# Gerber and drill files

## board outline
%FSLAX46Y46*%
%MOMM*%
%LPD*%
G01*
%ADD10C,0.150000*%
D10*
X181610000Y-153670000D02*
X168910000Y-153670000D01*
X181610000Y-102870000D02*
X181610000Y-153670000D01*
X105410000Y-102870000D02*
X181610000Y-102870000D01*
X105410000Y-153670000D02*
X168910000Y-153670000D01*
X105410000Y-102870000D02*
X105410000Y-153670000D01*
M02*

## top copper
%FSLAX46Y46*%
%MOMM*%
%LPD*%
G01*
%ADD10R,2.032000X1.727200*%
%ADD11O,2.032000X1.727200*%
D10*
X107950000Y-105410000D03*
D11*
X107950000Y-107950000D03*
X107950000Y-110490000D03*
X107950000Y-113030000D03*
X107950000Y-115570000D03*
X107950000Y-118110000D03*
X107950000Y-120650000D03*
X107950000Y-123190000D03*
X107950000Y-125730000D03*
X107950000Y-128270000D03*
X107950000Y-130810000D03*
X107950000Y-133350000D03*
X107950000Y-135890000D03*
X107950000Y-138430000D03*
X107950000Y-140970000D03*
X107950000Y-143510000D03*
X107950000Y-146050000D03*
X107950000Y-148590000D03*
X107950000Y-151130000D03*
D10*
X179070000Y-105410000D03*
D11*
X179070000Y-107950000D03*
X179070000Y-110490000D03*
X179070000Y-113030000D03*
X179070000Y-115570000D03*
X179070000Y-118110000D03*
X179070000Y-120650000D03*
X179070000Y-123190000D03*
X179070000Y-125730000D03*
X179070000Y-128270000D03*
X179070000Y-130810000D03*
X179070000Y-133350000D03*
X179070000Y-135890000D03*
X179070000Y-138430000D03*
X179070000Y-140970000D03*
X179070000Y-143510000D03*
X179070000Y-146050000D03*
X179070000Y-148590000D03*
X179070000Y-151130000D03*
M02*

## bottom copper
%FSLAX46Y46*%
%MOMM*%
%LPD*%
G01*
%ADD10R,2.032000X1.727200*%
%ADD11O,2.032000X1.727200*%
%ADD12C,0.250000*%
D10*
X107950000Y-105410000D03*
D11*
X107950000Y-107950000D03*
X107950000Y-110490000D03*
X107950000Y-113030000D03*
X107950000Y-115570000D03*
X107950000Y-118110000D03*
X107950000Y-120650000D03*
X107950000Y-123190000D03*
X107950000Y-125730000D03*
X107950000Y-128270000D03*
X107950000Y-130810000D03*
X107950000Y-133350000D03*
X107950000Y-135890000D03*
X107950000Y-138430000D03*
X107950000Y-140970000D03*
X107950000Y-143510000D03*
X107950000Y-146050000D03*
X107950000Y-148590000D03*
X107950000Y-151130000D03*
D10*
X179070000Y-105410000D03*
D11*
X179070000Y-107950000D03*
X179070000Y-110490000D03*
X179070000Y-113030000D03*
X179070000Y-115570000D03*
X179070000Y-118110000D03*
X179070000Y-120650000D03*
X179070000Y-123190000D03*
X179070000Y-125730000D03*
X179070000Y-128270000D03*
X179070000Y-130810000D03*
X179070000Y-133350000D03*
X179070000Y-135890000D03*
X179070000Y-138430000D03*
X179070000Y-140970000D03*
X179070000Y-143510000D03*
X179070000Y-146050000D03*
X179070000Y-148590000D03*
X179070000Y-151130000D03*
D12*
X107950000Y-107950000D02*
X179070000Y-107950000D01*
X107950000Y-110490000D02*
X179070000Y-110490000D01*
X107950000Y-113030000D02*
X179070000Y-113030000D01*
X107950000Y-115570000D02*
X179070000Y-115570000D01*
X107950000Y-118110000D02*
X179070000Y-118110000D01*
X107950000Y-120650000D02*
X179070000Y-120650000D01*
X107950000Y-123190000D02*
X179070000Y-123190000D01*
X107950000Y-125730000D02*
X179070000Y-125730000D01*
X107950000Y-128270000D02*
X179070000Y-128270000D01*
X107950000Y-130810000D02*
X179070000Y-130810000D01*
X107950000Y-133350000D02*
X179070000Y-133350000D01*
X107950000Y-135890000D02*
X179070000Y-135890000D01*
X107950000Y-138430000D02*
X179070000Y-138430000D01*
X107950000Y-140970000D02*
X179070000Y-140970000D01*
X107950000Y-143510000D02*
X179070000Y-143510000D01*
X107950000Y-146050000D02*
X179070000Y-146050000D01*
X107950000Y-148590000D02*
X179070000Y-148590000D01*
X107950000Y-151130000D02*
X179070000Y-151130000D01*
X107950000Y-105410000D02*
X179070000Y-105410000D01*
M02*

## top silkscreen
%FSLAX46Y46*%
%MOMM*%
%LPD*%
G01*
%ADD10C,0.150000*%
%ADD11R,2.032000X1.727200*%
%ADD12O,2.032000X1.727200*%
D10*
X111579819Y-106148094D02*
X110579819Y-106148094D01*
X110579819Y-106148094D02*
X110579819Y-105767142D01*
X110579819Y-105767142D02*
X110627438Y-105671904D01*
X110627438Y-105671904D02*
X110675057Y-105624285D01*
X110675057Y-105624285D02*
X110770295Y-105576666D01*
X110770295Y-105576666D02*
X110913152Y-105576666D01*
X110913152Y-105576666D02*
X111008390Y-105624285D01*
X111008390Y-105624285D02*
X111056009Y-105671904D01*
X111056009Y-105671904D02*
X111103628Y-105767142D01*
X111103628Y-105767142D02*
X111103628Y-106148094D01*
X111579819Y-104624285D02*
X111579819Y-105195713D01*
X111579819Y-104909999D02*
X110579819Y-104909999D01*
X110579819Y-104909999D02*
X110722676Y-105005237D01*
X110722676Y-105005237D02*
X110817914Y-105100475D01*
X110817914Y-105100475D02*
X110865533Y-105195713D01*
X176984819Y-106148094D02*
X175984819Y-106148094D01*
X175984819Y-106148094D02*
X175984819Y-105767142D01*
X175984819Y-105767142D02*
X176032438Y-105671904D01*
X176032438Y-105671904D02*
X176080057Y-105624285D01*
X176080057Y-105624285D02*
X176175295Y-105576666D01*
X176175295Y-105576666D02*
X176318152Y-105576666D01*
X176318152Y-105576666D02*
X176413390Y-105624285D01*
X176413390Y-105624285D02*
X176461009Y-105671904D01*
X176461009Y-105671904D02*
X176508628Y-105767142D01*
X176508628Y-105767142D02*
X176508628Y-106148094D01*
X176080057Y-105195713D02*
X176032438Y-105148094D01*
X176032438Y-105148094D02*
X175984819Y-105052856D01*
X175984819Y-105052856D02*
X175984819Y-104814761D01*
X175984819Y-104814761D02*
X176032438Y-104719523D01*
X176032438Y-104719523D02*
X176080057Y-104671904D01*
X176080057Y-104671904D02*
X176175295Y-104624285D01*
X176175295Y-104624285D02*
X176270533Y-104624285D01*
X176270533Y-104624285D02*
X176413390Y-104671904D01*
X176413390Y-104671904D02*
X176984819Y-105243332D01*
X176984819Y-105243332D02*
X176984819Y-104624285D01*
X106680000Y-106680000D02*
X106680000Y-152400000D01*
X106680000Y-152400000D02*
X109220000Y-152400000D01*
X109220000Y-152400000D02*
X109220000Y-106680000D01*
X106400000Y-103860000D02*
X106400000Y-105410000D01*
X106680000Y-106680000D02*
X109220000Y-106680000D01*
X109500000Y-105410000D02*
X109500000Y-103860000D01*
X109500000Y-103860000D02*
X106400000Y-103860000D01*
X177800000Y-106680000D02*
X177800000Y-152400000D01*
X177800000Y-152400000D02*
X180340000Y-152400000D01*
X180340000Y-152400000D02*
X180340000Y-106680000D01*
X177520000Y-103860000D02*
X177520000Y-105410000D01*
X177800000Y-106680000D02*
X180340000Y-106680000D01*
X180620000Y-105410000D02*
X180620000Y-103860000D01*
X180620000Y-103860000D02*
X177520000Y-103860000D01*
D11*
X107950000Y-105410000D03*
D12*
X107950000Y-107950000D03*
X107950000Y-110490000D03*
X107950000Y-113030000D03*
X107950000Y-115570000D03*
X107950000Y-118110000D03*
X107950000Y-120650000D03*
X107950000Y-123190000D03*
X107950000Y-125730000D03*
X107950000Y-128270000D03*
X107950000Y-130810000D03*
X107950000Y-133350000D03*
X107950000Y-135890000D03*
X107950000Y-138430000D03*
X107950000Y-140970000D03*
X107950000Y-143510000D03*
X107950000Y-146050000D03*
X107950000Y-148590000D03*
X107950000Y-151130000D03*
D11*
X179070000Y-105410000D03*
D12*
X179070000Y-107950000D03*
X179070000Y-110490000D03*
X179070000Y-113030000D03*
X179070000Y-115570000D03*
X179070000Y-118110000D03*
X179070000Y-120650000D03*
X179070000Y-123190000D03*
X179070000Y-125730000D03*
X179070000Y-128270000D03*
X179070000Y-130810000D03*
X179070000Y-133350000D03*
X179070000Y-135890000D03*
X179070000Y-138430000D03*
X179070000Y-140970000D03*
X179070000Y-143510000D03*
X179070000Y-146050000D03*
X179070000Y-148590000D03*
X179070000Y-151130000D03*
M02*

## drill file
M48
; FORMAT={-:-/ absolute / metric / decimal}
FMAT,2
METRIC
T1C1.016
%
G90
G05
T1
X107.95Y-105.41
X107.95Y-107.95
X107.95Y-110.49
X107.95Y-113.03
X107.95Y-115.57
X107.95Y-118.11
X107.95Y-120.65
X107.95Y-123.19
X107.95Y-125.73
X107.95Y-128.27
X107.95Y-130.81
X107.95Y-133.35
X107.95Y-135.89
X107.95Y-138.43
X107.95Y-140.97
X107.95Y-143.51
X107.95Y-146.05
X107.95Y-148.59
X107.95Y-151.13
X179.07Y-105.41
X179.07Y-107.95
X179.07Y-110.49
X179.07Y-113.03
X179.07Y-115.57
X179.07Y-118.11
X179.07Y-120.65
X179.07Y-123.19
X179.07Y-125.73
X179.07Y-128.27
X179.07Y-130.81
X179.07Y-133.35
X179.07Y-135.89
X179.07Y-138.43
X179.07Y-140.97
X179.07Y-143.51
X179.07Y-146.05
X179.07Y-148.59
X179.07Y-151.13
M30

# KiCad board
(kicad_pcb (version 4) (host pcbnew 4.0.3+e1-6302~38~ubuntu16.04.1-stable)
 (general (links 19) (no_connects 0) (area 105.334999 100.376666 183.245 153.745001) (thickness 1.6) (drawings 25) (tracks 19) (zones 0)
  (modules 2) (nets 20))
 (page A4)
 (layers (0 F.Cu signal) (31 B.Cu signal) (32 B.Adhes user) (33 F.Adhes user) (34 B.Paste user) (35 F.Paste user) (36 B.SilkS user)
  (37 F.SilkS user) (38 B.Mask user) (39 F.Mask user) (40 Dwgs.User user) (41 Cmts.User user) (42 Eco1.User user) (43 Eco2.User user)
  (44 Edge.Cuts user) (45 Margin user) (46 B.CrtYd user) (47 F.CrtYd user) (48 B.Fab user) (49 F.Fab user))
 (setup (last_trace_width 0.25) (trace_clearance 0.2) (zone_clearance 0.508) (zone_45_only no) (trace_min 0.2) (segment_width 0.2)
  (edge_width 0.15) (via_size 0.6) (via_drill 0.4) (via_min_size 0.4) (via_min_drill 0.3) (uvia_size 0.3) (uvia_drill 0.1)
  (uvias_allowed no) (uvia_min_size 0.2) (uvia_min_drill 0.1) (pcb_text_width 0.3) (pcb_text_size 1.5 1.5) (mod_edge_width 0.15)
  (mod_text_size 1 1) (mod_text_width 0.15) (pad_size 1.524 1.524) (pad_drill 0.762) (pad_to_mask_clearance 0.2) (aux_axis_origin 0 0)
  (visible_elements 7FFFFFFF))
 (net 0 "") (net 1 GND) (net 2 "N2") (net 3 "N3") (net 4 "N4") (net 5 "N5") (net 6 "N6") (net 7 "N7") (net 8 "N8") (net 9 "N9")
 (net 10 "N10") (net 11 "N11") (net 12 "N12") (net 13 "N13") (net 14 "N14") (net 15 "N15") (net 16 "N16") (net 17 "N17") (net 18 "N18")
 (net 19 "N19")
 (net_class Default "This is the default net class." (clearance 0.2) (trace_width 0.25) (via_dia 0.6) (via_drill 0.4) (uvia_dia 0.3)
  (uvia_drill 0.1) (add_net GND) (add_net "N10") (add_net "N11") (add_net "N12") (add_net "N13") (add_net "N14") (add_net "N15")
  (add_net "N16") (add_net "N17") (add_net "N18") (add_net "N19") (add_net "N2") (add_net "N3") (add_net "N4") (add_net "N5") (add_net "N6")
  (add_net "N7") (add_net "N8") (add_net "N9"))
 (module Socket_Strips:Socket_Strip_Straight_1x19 (layer F.Cu) (at 107.95 105.41 270)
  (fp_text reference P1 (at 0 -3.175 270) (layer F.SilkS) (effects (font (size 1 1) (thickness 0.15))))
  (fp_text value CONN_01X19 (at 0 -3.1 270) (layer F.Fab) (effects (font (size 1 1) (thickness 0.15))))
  (fp_line (start 1.27 1.27) (end 46.99 1.27) (layer F.SilkS) (width 0.15))
  (fp_line (start 46.99 1.27) (end 46.99 -1.27) (layer F.SilkS) (width 0.15))
  (fp_line (start 46.99 -1.27) (end 1.27 -1.27) (layer F.SilkS) (width 0.15))
  (fp_line (start -1.55 1.55) (end 0 1.55) (layer F.SilkS) (width 0.15))
  (fp_line (start 1.27 1.27) (end 1.27 -1.27) (layer F.SilkS) (width 0.15))
  (fp_line (start 0 -1.55) (end -1.55 -1.55) (layer F.SilkS) (width 0.15))
  (fp_line (start -1.55 -1.55) (end -1.55 1.55) (layer F.SilkS) (width 0.15))
  (pad 1 thru_hole rect (at 0 0 270) (size 1.7272 2.032) (drill 1.016) (layers *.Cu *.Mask F.SilkS) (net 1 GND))
  (pad 2 thru_hole oval (at 2.54 0 270) (size 1.7272 2.032) (drill 1.016) (layers *.Cu *.Mask F.SilkS) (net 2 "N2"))
  (pad 3 thru_hole oval (at 5.08 0 270) (size 1.7272 2.032) (drill 1.016) (layers *.Cu *.Mask F.SilkS) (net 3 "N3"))
  (pad 4 thru_hole oval (at 7.62 0 270) (size 1.7272 2.032) (drill 1.016) (layers *.Cu *.Mask F.SilkS) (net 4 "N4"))
  (pad 5 thru_hole oval (at 10.16 0 270) (size 1.7272 2.032) (drill 1.016) (layers *.Cu *.Mask F.SilkS) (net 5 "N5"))
  (pad 6 thru_hole oval (at 12.7 0 270) (size 1.7272 2.032) (drill 1.016) (layers *.Cu *.Mask F.SilkS) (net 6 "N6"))
  (pad 7 thru_hole oval (at 15.24 0 270) (size 1.7272 2.032) (drill 1.016) (layers *.Cu *.Mask F.SilkS) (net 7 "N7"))
  (pad 8 thru_hole oval (at 17.78 0 270) (size 1.7272 2.032) (drill 1.016) (layers *.Cu *.Mask F.SilkS) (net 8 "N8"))
  (pad 9 thru_hole oval (at 20.32 0 270) (size 1.7272 2.032) (drill 1.016) (layers *.Cu *.Mask F.SilkS) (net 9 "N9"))
  (pad 10 thru_hole oval (at 22.86 0 270) (size 1.7272 2.032) (drill 1.016) (layers *.Cu *.Mask F.SilkS) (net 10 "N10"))
  (pad 11 thru_hole oval (at 25.4 0 270) (size 1.7272 2.032) (drill 1.016) (layers *.Cu *.Mask F.SilkS) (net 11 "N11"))
  (pad 12 thru_hole oval (at 27.94 0 270) (size 1.7272 2.032) (drill 1.016) (layers *.Cu *.Mask F.SilkS) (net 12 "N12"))
  (pad 13 thru_hole oval (at 30.48 0 270) (size 1.7272 2.032) (drill 1.016) (layers *.Cu *.Mask F.SilkS) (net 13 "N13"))
  (pad 14 thru_hole oval (at 33.02 0 270) (size 1.7272 2.032) (drill 1.016) (layers *.Cu *.Mask F.SilkS) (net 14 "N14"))
  (pad 15 thru_hole oval (at 35.56 0 270) (size 1.7272 2.032) (drill 1.016) (layers *.Cu *.Mask F.SilkS) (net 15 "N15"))
  (pad 16 thru_hole oval (at 38.1 0 270) (size 1.7272 2.032) (drill 1.016) (layers *.Cu *.Mask F.SilkS) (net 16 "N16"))
  (pad 17 thru_hole oval (at 40.64 0 270) (size 1.7272 2.032) (drill 1.016) (layers *.Cu *.Mask F.SilkS) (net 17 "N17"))
  (pad 18 thru_hole oval (at 43.18 0 270) (size 1.7272 2.032) (drill 1.016) (layers *.Cu *.Mask F.SilkS) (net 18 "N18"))
  (pad 19 thru_hole oval (at 45.72 0 270) (size 1.7272 2.032) (drill 1.016) (layers *.Cu *.Mask F.SilkS) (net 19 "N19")))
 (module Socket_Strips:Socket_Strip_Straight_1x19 (layer F.Cu) (at 179.07 105.41 270)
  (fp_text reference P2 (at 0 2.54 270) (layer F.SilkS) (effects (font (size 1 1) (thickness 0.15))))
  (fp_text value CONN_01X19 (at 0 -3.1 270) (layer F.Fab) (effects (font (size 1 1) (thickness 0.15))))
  (fp_line (start 1.27 1.27) (end 46.99 1.27) (layer F.SilkS) (width 0.15))
  (fp_line (start 46.99 1.27) (end 46.99 -1.27) (layer F.SilkS) (width 0.15))
  (fp_line (start 46.99 -1.27) (end 1.27 -1.27) (layer F.SilkS) (width 0.15))
  (fp_line (start -1.55 1.55) (end 0 1.55) (layer F.SilkS) (width 0.15))
  (fp_line (start 1.27 1.27) (end 1.27 -1.27) (layer F.SilkS) (width 0.15))
  (fp_line (start 0 -1.55) (end -1.55 -1.55) (layer F.SilkS) (width 0.15))
  (fp_line (start -1.55 -1.55) (end -1.55 1.55) (layer F.SilkS) (width 0.15))
  (pad 1 thru_hole rect (at 0 0 270) (size 1.7272 2.032) (drill 1.016) (layers *.Cu *.Mask F.SilkS) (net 1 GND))
  (pad 2 thru_hole oval (at 2.54 0 270) (size 1.7272 2.032) (drill 1.016) (layers *.Cu *.Mask F.SilkS) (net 2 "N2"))
  (pad 3 thru_hole oval (at 5.08 0 270) (size 1.7272 2.032) (drill 1.016) (layers *.Cu *.Mask F.SilkS) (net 3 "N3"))
  (pad 4 thru_hole oval (at 7.62 0 270) (size 1.7272 2.032) (drill 1.016) (layers *.Cu *.Mask F.SilkS) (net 4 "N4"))
  (pad 5 thru_hole oval (at 10.16 0 270) (size 1.7272 2.032) (drill 1.016) (layers *.Cu *.Mask F.SilkS) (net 5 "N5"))
  (pad 6 thru_hole oval (at 12.7 0 270) (size 1.7272 2.032) (drill 1.016) (layers *.Cu *.Mask F.SilkS) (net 6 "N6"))
  (pad 7 thru_hole oval (at 15.24 0 270) (size 1.7272 2.032) (drill 1.016) (layers *.Cu *.Mask F.SilkS) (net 7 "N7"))
  (pad 8 thru_hole oval (at 17.78 0 270) (size 1.7272 2.032) (drill 1.016) (layers *.Cu *.Mask F.SilkS) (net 8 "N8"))
  (pad 9 thru_hole oval (at 20.32 0 270) (size 1.7272 2.032) (drill 1.016) (layers *.Cu *.Mask F.SilkS) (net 9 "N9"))
  (pad 10 thru_hole oval (at 22.86 0 270) (size 1.7272 2.032) (drill 1.016) (layers *.Cu *.Mask F.SilkS) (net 10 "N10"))
  (pad 11 thru_hole oval (at 25.4 0 270) (size 1.7272 2.032) (drill 1.016) (layers *.Cu *.Mask F.SilkS) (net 11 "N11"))
  (pad 12 thru_hole oval (at 27.94 0 270) (size 1.7272 2.032) (drill 1.016) (layers *.Cu *.Mask F.SilkS) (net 12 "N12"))
  (pad 13 thru_hole oval (at 30.48 0 270) (size 1.7272 2.032) (drill 1.016) (layers *.Cu *.Mask F.SilkS) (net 13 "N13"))
  (pad 14 thru_hole oval (at 33.02 0 270) (size 1.7272 2.032) (drill 1.016) (layers *.Cu *.Mask F.SilkS) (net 14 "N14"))
  (pad 15 thru_hole oval (at 35.56 0 270) (size 1.7272 2.032) (drill 1.016) (layers *.Cu *.Mask F.SilkS) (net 15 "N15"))
  (pad 16 thru_hole oval (at 38.1 0 270) (size 1.7272 2.032) (drill 1.016) (layers *.Cu *.Mask F.SilkS) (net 16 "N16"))
  (pad 17 thru_hole oval (at 40.64 0 270) (size 1.7272 2.032) (drill 1.016) (layers *.Cu *.Mask F.SilkS) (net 17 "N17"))
  (pad 18 thru_hole oval (at 43.18 0 270) (size 1.7272 2.032) (drill 1.016) (layers *.Cu *.Mask F.SilkS) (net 18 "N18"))
  (pad 19 thru_hole oval (at 45.72 0 270) (size 1.7272 2.032) (drill 1.016) (layers *.Cu *.Mask F.SilkS) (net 19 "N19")))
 (gr_line (start 181.61 153.67) (end 168.91 153.67) (angle 90) (layer Edge.Cuts) (width 0.15))
 (gr_line (start 181.61 102.87) (end 181.61 153.67) (angle 90) (layer Edge.Cuts) (width 0.15))
 (gr_line (start 105.41 102.87) (end 181.61 102.87) (angle 90) (layer Edge.Cuts) (width 0.15))
 (gr_line (start 105.41 153.67) (end 168.91 153.67) (angle 90) (layer Edge.Cuts) (width 0.15))
 (gr_line (start 105.41 102.87) (end 105.41 153.67) (angle 90) (layer Edge.Cuts) (width 0.15))
 (segment (start 107.95 107.95) (end 179.07 107.95) (width 0.25) (layer B.Cu) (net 2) (status 20))
 (segment (start 107.95 110.49) (end 179.07 110.49) (width 0.25) (layer B.Cu) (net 3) (status 20))
 (segment (start 107.95 113.03) (end 179.07 113.03) (width 0.25) (layer B.Cu) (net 4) (status 20))
 (segment (start 107.95 115.57) (end 179.07 115.57) (width 0.25) (layer B.Cu) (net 5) (status 20))
 (segment (start 107.95 118.11) (end 179.07 118.11) (width 0.25) (layer B.Cu) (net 6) (status 20))
 (segment (start 107.95 120.65) (end 179.07 120.65) (width 0.25) (layer B.Cu) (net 7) (status 20))
 (segment (start 107.95 123.19) (end 179.07 123.19) (width 0.25) (layer B.Cu) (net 8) (status 20))
 (segment (start 107.95 125.73) (end 179.07 125.73) (width 0.25) (layer B.Cu) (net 9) (status 20))
 (segment (start 107.95 128.27) (end 179.07 128.27) (width 0.25) (layer B.Cu) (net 10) (status 20))
 (segment (start 107.95 130.81) (end 179.07 130.81) (width 0.25) (layer B.Cu) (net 11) (status 20))
 (segment (start 107.95 133.35) (end 179.07 133.35) (width 0.25) (layer B.Cu) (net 12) (status 20))
 (segment (start 107.95 135.89) (end 179.07 135.89) (width 0.25) (layer B.Cu) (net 13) (status 20))
 (segment (start 107.95 138.43) (end 179.07 138.43) (width 0.25) (layer B.Cu) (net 14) (status 20))
 (segment (start 107.95 140.97) (end 179.07 140.97) (width 0.25) (layer B.Cu) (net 15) (status 20))
 (segment (start 107.95 143.51) (end 179.07 143.51) (width 0.25) (layer B.Cu) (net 16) (status 20))
 (segment (start 107.95 146.05) (end 179.07 146.05) (width 0.25) (layer B.Cu) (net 17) (status 20))
 (segment (start 107.95 148.59) (end 179.07 148.59) (width 0.25) (layer B.Cu) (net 18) (status 20))
 (segment (start 107.95 151.13) (end 179.07 151.13) (width 0.25) (layer B.Cu) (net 19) (status 20))
 (segment (start 107.95 105.41) (end 179.07 105.41) (width 0.25) (layer B.Cu) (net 1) (status 20)))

